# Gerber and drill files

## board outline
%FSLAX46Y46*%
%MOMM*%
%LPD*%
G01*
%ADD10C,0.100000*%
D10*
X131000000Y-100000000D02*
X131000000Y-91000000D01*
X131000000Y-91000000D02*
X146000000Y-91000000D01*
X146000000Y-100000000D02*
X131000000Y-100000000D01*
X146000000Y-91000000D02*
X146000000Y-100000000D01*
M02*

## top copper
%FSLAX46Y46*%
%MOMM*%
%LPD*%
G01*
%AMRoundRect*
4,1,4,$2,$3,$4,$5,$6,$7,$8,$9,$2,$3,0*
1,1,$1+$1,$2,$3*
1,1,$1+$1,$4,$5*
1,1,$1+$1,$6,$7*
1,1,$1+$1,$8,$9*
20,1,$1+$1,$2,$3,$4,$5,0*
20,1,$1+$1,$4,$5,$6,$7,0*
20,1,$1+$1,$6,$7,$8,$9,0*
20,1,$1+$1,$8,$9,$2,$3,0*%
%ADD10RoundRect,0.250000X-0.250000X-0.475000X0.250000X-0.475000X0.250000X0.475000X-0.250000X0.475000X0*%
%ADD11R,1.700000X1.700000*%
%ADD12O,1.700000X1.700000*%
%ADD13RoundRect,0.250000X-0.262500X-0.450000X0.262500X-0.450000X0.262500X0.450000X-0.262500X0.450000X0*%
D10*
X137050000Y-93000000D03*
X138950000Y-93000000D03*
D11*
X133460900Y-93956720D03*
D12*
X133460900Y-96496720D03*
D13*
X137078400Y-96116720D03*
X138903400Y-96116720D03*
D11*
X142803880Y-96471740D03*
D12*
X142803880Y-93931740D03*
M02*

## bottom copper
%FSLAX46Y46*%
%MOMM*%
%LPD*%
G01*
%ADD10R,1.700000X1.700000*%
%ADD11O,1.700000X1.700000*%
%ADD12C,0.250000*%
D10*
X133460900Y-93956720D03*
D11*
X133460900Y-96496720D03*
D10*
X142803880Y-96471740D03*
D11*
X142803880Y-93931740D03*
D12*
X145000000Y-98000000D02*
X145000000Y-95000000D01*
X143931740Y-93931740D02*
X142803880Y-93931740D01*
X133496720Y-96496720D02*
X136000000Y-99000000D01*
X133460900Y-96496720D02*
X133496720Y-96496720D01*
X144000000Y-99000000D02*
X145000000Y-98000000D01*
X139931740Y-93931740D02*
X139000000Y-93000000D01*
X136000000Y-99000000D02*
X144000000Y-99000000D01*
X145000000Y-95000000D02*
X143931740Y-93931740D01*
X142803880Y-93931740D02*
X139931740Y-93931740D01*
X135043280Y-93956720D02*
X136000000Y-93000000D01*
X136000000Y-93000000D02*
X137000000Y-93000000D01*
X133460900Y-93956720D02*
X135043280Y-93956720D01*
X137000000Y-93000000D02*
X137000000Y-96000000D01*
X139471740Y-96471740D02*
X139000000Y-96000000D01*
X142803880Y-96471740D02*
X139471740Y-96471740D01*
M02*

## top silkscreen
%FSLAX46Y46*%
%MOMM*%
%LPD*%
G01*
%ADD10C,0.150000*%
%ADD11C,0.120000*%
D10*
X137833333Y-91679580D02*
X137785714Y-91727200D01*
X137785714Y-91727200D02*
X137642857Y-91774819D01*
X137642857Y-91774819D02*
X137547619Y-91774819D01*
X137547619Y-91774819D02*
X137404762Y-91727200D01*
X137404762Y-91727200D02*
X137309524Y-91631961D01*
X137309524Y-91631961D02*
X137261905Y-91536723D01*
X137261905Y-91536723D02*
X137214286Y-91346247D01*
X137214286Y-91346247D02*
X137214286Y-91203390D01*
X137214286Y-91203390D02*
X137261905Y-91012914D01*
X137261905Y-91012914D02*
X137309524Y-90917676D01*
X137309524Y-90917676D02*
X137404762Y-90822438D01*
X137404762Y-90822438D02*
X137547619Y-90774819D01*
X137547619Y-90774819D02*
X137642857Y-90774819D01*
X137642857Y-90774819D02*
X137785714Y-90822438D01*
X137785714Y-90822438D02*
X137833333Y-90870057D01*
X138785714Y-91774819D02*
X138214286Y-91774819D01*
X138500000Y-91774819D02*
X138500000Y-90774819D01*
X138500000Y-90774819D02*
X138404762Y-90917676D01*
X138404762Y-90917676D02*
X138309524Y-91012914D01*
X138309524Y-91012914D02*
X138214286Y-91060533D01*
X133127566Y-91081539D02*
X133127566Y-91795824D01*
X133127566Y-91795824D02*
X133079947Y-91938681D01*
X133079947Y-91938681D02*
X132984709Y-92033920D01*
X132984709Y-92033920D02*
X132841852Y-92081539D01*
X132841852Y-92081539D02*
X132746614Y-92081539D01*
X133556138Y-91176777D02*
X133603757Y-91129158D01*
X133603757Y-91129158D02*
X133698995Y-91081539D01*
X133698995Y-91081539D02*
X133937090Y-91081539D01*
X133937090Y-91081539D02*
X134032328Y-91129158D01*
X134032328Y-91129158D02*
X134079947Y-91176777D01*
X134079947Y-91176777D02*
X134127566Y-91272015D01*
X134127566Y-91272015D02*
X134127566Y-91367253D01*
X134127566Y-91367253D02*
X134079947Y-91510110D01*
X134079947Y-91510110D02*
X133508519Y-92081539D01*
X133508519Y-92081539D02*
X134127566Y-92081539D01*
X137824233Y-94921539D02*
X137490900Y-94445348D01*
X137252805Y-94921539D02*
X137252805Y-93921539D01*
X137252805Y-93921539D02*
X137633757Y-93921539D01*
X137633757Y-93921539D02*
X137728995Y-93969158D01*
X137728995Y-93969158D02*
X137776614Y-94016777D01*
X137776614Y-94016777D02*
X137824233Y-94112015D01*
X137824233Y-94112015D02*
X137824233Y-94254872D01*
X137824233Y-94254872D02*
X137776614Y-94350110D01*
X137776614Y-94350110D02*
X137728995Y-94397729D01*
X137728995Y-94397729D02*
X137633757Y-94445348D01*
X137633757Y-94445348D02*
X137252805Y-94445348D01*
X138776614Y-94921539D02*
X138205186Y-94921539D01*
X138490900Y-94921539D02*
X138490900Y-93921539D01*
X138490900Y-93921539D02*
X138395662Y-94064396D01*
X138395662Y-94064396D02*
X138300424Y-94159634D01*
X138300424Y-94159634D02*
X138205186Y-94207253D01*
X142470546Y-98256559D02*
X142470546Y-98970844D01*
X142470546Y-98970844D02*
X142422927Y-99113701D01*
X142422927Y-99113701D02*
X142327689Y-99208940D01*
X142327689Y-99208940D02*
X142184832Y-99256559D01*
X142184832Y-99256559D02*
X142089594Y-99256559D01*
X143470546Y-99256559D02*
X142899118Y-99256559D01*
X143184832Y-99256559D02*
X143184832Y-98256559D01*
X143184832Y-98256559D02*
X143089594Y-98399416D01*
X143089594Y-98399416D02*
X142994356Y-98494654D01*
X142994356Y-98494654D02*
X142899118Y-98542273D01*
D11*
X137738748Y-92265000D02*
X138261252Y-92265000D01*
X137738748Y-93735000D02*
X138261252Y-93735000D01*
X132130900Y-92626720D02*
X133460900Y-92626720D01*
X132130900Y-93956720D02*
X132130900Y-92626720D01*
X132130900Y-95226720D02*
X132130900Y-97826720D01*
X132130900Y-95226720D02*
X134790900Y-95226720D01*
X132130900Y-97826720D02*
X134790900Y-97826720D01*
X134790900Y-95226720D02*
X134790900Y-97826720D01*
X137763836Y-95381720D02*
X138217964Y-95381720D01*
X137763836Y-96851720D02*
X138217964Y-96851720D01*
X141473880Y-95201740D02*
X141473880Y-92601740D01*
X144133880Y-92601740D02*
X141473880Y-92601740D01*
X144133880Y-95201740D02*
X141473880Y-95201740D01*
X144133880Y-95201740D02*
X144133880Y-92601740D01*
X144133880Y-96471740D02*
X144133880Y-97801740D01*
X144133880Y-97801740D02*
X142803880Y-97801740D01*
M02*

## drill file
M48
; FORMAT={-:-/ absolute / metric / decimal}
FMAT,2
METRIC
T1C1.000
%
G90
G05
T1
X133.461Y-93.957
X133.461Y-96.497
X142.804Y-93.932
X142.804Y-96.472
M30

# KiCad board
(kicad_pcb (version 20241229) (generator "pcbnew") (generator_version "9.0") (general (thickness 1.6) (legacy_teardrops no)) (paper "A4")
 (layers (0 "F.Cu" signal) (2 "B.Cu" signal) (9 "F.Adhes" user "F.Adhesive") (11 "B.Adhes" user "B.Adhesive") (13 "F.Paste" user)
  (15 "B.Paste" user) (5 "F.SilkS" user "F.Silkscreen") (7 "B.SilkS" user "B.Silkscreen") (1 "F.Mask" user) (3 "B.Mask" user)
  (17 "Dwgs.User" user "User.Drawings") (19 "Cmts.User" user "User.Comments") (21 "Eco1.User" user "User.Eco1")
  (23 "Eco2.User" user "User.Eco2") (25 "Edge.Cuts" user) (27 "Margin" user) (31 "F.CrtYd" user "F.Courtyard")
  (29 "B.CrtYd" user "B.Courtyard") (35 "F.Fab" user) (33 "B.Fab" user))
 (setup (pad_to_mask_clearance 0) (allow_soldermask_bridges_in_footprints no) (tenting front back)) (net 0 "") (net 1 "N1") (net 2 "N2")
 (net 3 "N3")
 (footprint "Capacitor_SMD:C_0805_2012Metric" (layer "F.Cu") (at 138 93)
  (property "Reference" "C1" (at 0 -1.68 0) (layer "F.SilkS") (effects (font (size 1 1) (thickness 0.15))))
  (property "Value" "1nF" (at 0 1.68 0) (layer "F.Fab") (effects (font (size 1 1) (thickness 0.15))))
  (fp_line (start -0.261252 -0.735) (end 0.261252 -0.735) (stroke (width 0.12) (type solid)) (layer "F.SilkS"))
  (fp_line (start -0.261252 0.735) (end 0.261252 0.735) (stroke (width 0.12) (type solid)) (layer "F.SilkS"))
  (pad "1" smd roundrect (at -0.95 0) (size 1 1.45) (layers "F.Cu" "F.Mask" "F.Paste") (roundrect_rratio 0.25) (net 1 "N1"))
  (pad "2" smd roundrect (at 0.95 0) (size 1 1.45) (layers "F.Cu" "F.Mask" "F.Paste") (roundrect_rratio 0.25) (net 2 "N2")))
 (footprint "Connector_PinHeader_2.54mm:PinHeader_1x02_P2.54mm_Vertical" (layer "F.Cu") (at 133.4609 93.95672)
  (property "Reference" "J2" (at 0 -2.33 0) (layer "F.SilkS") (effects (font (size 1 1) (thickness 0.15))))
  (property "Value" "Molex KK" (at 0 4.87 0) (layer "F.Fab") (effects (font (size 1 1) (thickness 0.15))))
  (fp_line (start -1.33 -1.33) (end 0 -1.33) (stroke (width 0.12) (type solid)) (layer "F.SilkS"))
  (fp_line (start -1.33 0) (end -1.33 -1.33) (stroke (width 0.12) (type solid)) (layer "F.SilkS"))
  (fp_line (start -1.33 1.27) (end -1.33 3.87) (stroke (width 0.12) (type solid)) (layer "F.SilkS"))
  (fp_line (start -1.33 1.27) (end 1.33 1.27) (stroke (width 0.12) (type solid)) (layer "F.SilkS"))
  (fp_line (start -1.33 3.87) (end 1.33 3.87) (stroke (width 0.12) (type solid)) (layer "F.SilkS"))
  (fp_line (start 1.33 1.27) (end 1.33 3.87) (stroke (width 0.12) (type solid)) (layer "F.SilkS"))
  (pad "1" thru_hole rect (at 0 0) (size 1.7 1.7) (drill 1) (layers "*.Cu" "*.Mask") (remove_unused_layers no) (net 1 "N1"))
  (pad "2" thru_hole oval (at 0 2.54) (size 1.7 1.7) (drill 1) (layers "*.Cu" "*.Mask") (remove_unused_layers no) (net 2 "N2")))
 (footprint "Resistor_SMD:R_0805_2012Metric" (layer "F.Cu") (at 137.9909 96.11672)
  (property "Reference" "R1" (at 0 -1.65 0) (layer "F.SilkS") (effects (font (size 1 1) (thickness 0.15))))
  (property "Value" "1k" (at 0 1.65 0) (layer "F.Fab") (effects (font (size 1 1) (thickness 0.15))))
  (fp_line (start -0.227064 -0.735) (end 0.227064 -0.735) (stroke (width 0.12) (type solid)) (layer "F.SilkS"))
  (fp_line (start -0.227064 0.735) (end 0.227064 0.735) (stroke (width 0.12) (type solid)) (layer "F.SilkS"))
  (pad "1" smd roundrect (at -0.9125 0) (size 1.025 1.4) (layers "F.Cu" "F.Mask" "F.Paste") (roundrect_rratio 0.243902) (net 1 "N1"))
  (pad "2" smd roundrect (at 0.9125 0) (size 1.025 1.4) (layers "F.Cu" "F.Mask" "F.Paste") (roundrect_rratio 0.243902) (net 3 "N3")))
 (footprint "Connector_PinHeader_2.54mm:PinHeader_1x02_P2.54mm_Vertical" (layer "F.Cu") (at 142.80388 96.47174 180)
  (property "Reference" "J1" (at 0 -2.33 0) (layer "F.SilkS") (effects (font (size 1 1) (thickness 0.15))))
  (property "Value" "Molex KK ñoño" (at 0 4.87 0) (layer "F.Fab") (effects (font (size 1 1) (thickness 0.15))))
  (fp_line (start 1.33 1.27) (end 1.33 3.87) (stroke (width 0.12) (type solid)) (layer "F.SilkS"))
  (fp_line (start -1.33 3.87) (end 1.33 3.87) (stroke (width 0.12) (type solid)) (layer "F.SilkS"))
  (fp_line (start -1.33 1.27) (end 1.33 1.27) (stroke (width 0.12) (type solid)) (layer "F.SilkS"))
  (fp_line (start -1.33 1.27) (end -1.33 3.87) (stroke (width 0.12) (type solid)) (layer "F.SilkS"))
  (fp_line (start -1.33 0) (end -1.33 -1.33) (stroke (width 0.12) (type solid)) (layer "F.SilkS"))
  (fp_line (start -1.33 -1.33) (end 0 -1.33) (stroke (width 0.12) (type solid)) (layer "F.SilkS"))
  (pad "1" thru_hole rect (at 0 0 180) (size 1.7 1.7) (drill 1) (layers "*.Cu" "*.Mask") (remove_unused_layers no) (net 3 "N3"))
  (pad "2" thru_hole oval (at 0 2.54 180) (size 1.7 1.7) (drill 1) (layers "*.Cu" "*.Mask") (remove_unused_layers no) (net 2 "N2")))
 (gr_line (start 131 100) (end 131 91) (stroke (width 0.1) (type solid)) (layer "Edge.Cuts"))
 (gr_line (start 131 91) (end 146 91) (stroke (width 0.1) (type solid)) (layer "Edge.Cuts"))
 (gr_line (start 146 100) (end 131 100) (stroke (width 0.1) (type solid)) (layer "Edge.Cuts"))
 (gr_line (start 146 91) (end 146 100) (stroke (width 0.1) (type solid)) (layer "Edge.Cuts"))
 (segment (start 145 98) (end 145 95) (width 0.25) (layer "B.Cu") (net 2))
 (segment (start 143.93174 93.93174) (end 142.80388 93.93174) (width 0.25) (layer "B.Cu") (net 2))
 (segment (start 133.49672 96.49672) (end 136 99) (width 0.25) (layer "B.Cu") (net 2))
 (segment (start 133.4609 96.49672) (end 133.49672 96.49672) (width 0.25) (layer "B.Cu") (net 2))
 (segment (start 144 99) (end 145 98) (width 0.25) (layer "B.Cu") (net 2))
 (segment (start 139.93174 93.93174) (end 139 93) (width 0.25) (layer "B.Cu") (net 2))
 (segment (start 136 99) (end 144 99) (width 0.25) (layer "B.Cu") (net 2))
 (segment (start 145 95) (end 143.93174 93.93174) (width 0.25) (layer "B.Cu") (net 2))
 (segment (start 142.80388 93.93174) (end 139.93174 93.93174) (width 0.25) (layer "B.Cu") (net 2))
 (segment (start 135.04328 93.95672) (end 136 93) (width 0.25) (layer "B.Cu") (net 1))
 (segment (start 136 93) (end 137 93) (width 0.25) (layer "B.Cu") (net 1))
 (segment (start 133.4609 93.95672) (end 135.04328 93.95672) (width 0.25) (layer "B.Cu") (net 1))
 (segment (start 137 93) (end 137 96) (width 0.25) (layer "B.Cu") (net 1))
 (segment (start 139.47174 96.47174) (end 139 96) (width 0.25) (layer "B.Cu") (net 3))
 (segment (start 142.80388 96.47174) (end 139.47174 96.47174) (width 0.25) (layer "B.Cu") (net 3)))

